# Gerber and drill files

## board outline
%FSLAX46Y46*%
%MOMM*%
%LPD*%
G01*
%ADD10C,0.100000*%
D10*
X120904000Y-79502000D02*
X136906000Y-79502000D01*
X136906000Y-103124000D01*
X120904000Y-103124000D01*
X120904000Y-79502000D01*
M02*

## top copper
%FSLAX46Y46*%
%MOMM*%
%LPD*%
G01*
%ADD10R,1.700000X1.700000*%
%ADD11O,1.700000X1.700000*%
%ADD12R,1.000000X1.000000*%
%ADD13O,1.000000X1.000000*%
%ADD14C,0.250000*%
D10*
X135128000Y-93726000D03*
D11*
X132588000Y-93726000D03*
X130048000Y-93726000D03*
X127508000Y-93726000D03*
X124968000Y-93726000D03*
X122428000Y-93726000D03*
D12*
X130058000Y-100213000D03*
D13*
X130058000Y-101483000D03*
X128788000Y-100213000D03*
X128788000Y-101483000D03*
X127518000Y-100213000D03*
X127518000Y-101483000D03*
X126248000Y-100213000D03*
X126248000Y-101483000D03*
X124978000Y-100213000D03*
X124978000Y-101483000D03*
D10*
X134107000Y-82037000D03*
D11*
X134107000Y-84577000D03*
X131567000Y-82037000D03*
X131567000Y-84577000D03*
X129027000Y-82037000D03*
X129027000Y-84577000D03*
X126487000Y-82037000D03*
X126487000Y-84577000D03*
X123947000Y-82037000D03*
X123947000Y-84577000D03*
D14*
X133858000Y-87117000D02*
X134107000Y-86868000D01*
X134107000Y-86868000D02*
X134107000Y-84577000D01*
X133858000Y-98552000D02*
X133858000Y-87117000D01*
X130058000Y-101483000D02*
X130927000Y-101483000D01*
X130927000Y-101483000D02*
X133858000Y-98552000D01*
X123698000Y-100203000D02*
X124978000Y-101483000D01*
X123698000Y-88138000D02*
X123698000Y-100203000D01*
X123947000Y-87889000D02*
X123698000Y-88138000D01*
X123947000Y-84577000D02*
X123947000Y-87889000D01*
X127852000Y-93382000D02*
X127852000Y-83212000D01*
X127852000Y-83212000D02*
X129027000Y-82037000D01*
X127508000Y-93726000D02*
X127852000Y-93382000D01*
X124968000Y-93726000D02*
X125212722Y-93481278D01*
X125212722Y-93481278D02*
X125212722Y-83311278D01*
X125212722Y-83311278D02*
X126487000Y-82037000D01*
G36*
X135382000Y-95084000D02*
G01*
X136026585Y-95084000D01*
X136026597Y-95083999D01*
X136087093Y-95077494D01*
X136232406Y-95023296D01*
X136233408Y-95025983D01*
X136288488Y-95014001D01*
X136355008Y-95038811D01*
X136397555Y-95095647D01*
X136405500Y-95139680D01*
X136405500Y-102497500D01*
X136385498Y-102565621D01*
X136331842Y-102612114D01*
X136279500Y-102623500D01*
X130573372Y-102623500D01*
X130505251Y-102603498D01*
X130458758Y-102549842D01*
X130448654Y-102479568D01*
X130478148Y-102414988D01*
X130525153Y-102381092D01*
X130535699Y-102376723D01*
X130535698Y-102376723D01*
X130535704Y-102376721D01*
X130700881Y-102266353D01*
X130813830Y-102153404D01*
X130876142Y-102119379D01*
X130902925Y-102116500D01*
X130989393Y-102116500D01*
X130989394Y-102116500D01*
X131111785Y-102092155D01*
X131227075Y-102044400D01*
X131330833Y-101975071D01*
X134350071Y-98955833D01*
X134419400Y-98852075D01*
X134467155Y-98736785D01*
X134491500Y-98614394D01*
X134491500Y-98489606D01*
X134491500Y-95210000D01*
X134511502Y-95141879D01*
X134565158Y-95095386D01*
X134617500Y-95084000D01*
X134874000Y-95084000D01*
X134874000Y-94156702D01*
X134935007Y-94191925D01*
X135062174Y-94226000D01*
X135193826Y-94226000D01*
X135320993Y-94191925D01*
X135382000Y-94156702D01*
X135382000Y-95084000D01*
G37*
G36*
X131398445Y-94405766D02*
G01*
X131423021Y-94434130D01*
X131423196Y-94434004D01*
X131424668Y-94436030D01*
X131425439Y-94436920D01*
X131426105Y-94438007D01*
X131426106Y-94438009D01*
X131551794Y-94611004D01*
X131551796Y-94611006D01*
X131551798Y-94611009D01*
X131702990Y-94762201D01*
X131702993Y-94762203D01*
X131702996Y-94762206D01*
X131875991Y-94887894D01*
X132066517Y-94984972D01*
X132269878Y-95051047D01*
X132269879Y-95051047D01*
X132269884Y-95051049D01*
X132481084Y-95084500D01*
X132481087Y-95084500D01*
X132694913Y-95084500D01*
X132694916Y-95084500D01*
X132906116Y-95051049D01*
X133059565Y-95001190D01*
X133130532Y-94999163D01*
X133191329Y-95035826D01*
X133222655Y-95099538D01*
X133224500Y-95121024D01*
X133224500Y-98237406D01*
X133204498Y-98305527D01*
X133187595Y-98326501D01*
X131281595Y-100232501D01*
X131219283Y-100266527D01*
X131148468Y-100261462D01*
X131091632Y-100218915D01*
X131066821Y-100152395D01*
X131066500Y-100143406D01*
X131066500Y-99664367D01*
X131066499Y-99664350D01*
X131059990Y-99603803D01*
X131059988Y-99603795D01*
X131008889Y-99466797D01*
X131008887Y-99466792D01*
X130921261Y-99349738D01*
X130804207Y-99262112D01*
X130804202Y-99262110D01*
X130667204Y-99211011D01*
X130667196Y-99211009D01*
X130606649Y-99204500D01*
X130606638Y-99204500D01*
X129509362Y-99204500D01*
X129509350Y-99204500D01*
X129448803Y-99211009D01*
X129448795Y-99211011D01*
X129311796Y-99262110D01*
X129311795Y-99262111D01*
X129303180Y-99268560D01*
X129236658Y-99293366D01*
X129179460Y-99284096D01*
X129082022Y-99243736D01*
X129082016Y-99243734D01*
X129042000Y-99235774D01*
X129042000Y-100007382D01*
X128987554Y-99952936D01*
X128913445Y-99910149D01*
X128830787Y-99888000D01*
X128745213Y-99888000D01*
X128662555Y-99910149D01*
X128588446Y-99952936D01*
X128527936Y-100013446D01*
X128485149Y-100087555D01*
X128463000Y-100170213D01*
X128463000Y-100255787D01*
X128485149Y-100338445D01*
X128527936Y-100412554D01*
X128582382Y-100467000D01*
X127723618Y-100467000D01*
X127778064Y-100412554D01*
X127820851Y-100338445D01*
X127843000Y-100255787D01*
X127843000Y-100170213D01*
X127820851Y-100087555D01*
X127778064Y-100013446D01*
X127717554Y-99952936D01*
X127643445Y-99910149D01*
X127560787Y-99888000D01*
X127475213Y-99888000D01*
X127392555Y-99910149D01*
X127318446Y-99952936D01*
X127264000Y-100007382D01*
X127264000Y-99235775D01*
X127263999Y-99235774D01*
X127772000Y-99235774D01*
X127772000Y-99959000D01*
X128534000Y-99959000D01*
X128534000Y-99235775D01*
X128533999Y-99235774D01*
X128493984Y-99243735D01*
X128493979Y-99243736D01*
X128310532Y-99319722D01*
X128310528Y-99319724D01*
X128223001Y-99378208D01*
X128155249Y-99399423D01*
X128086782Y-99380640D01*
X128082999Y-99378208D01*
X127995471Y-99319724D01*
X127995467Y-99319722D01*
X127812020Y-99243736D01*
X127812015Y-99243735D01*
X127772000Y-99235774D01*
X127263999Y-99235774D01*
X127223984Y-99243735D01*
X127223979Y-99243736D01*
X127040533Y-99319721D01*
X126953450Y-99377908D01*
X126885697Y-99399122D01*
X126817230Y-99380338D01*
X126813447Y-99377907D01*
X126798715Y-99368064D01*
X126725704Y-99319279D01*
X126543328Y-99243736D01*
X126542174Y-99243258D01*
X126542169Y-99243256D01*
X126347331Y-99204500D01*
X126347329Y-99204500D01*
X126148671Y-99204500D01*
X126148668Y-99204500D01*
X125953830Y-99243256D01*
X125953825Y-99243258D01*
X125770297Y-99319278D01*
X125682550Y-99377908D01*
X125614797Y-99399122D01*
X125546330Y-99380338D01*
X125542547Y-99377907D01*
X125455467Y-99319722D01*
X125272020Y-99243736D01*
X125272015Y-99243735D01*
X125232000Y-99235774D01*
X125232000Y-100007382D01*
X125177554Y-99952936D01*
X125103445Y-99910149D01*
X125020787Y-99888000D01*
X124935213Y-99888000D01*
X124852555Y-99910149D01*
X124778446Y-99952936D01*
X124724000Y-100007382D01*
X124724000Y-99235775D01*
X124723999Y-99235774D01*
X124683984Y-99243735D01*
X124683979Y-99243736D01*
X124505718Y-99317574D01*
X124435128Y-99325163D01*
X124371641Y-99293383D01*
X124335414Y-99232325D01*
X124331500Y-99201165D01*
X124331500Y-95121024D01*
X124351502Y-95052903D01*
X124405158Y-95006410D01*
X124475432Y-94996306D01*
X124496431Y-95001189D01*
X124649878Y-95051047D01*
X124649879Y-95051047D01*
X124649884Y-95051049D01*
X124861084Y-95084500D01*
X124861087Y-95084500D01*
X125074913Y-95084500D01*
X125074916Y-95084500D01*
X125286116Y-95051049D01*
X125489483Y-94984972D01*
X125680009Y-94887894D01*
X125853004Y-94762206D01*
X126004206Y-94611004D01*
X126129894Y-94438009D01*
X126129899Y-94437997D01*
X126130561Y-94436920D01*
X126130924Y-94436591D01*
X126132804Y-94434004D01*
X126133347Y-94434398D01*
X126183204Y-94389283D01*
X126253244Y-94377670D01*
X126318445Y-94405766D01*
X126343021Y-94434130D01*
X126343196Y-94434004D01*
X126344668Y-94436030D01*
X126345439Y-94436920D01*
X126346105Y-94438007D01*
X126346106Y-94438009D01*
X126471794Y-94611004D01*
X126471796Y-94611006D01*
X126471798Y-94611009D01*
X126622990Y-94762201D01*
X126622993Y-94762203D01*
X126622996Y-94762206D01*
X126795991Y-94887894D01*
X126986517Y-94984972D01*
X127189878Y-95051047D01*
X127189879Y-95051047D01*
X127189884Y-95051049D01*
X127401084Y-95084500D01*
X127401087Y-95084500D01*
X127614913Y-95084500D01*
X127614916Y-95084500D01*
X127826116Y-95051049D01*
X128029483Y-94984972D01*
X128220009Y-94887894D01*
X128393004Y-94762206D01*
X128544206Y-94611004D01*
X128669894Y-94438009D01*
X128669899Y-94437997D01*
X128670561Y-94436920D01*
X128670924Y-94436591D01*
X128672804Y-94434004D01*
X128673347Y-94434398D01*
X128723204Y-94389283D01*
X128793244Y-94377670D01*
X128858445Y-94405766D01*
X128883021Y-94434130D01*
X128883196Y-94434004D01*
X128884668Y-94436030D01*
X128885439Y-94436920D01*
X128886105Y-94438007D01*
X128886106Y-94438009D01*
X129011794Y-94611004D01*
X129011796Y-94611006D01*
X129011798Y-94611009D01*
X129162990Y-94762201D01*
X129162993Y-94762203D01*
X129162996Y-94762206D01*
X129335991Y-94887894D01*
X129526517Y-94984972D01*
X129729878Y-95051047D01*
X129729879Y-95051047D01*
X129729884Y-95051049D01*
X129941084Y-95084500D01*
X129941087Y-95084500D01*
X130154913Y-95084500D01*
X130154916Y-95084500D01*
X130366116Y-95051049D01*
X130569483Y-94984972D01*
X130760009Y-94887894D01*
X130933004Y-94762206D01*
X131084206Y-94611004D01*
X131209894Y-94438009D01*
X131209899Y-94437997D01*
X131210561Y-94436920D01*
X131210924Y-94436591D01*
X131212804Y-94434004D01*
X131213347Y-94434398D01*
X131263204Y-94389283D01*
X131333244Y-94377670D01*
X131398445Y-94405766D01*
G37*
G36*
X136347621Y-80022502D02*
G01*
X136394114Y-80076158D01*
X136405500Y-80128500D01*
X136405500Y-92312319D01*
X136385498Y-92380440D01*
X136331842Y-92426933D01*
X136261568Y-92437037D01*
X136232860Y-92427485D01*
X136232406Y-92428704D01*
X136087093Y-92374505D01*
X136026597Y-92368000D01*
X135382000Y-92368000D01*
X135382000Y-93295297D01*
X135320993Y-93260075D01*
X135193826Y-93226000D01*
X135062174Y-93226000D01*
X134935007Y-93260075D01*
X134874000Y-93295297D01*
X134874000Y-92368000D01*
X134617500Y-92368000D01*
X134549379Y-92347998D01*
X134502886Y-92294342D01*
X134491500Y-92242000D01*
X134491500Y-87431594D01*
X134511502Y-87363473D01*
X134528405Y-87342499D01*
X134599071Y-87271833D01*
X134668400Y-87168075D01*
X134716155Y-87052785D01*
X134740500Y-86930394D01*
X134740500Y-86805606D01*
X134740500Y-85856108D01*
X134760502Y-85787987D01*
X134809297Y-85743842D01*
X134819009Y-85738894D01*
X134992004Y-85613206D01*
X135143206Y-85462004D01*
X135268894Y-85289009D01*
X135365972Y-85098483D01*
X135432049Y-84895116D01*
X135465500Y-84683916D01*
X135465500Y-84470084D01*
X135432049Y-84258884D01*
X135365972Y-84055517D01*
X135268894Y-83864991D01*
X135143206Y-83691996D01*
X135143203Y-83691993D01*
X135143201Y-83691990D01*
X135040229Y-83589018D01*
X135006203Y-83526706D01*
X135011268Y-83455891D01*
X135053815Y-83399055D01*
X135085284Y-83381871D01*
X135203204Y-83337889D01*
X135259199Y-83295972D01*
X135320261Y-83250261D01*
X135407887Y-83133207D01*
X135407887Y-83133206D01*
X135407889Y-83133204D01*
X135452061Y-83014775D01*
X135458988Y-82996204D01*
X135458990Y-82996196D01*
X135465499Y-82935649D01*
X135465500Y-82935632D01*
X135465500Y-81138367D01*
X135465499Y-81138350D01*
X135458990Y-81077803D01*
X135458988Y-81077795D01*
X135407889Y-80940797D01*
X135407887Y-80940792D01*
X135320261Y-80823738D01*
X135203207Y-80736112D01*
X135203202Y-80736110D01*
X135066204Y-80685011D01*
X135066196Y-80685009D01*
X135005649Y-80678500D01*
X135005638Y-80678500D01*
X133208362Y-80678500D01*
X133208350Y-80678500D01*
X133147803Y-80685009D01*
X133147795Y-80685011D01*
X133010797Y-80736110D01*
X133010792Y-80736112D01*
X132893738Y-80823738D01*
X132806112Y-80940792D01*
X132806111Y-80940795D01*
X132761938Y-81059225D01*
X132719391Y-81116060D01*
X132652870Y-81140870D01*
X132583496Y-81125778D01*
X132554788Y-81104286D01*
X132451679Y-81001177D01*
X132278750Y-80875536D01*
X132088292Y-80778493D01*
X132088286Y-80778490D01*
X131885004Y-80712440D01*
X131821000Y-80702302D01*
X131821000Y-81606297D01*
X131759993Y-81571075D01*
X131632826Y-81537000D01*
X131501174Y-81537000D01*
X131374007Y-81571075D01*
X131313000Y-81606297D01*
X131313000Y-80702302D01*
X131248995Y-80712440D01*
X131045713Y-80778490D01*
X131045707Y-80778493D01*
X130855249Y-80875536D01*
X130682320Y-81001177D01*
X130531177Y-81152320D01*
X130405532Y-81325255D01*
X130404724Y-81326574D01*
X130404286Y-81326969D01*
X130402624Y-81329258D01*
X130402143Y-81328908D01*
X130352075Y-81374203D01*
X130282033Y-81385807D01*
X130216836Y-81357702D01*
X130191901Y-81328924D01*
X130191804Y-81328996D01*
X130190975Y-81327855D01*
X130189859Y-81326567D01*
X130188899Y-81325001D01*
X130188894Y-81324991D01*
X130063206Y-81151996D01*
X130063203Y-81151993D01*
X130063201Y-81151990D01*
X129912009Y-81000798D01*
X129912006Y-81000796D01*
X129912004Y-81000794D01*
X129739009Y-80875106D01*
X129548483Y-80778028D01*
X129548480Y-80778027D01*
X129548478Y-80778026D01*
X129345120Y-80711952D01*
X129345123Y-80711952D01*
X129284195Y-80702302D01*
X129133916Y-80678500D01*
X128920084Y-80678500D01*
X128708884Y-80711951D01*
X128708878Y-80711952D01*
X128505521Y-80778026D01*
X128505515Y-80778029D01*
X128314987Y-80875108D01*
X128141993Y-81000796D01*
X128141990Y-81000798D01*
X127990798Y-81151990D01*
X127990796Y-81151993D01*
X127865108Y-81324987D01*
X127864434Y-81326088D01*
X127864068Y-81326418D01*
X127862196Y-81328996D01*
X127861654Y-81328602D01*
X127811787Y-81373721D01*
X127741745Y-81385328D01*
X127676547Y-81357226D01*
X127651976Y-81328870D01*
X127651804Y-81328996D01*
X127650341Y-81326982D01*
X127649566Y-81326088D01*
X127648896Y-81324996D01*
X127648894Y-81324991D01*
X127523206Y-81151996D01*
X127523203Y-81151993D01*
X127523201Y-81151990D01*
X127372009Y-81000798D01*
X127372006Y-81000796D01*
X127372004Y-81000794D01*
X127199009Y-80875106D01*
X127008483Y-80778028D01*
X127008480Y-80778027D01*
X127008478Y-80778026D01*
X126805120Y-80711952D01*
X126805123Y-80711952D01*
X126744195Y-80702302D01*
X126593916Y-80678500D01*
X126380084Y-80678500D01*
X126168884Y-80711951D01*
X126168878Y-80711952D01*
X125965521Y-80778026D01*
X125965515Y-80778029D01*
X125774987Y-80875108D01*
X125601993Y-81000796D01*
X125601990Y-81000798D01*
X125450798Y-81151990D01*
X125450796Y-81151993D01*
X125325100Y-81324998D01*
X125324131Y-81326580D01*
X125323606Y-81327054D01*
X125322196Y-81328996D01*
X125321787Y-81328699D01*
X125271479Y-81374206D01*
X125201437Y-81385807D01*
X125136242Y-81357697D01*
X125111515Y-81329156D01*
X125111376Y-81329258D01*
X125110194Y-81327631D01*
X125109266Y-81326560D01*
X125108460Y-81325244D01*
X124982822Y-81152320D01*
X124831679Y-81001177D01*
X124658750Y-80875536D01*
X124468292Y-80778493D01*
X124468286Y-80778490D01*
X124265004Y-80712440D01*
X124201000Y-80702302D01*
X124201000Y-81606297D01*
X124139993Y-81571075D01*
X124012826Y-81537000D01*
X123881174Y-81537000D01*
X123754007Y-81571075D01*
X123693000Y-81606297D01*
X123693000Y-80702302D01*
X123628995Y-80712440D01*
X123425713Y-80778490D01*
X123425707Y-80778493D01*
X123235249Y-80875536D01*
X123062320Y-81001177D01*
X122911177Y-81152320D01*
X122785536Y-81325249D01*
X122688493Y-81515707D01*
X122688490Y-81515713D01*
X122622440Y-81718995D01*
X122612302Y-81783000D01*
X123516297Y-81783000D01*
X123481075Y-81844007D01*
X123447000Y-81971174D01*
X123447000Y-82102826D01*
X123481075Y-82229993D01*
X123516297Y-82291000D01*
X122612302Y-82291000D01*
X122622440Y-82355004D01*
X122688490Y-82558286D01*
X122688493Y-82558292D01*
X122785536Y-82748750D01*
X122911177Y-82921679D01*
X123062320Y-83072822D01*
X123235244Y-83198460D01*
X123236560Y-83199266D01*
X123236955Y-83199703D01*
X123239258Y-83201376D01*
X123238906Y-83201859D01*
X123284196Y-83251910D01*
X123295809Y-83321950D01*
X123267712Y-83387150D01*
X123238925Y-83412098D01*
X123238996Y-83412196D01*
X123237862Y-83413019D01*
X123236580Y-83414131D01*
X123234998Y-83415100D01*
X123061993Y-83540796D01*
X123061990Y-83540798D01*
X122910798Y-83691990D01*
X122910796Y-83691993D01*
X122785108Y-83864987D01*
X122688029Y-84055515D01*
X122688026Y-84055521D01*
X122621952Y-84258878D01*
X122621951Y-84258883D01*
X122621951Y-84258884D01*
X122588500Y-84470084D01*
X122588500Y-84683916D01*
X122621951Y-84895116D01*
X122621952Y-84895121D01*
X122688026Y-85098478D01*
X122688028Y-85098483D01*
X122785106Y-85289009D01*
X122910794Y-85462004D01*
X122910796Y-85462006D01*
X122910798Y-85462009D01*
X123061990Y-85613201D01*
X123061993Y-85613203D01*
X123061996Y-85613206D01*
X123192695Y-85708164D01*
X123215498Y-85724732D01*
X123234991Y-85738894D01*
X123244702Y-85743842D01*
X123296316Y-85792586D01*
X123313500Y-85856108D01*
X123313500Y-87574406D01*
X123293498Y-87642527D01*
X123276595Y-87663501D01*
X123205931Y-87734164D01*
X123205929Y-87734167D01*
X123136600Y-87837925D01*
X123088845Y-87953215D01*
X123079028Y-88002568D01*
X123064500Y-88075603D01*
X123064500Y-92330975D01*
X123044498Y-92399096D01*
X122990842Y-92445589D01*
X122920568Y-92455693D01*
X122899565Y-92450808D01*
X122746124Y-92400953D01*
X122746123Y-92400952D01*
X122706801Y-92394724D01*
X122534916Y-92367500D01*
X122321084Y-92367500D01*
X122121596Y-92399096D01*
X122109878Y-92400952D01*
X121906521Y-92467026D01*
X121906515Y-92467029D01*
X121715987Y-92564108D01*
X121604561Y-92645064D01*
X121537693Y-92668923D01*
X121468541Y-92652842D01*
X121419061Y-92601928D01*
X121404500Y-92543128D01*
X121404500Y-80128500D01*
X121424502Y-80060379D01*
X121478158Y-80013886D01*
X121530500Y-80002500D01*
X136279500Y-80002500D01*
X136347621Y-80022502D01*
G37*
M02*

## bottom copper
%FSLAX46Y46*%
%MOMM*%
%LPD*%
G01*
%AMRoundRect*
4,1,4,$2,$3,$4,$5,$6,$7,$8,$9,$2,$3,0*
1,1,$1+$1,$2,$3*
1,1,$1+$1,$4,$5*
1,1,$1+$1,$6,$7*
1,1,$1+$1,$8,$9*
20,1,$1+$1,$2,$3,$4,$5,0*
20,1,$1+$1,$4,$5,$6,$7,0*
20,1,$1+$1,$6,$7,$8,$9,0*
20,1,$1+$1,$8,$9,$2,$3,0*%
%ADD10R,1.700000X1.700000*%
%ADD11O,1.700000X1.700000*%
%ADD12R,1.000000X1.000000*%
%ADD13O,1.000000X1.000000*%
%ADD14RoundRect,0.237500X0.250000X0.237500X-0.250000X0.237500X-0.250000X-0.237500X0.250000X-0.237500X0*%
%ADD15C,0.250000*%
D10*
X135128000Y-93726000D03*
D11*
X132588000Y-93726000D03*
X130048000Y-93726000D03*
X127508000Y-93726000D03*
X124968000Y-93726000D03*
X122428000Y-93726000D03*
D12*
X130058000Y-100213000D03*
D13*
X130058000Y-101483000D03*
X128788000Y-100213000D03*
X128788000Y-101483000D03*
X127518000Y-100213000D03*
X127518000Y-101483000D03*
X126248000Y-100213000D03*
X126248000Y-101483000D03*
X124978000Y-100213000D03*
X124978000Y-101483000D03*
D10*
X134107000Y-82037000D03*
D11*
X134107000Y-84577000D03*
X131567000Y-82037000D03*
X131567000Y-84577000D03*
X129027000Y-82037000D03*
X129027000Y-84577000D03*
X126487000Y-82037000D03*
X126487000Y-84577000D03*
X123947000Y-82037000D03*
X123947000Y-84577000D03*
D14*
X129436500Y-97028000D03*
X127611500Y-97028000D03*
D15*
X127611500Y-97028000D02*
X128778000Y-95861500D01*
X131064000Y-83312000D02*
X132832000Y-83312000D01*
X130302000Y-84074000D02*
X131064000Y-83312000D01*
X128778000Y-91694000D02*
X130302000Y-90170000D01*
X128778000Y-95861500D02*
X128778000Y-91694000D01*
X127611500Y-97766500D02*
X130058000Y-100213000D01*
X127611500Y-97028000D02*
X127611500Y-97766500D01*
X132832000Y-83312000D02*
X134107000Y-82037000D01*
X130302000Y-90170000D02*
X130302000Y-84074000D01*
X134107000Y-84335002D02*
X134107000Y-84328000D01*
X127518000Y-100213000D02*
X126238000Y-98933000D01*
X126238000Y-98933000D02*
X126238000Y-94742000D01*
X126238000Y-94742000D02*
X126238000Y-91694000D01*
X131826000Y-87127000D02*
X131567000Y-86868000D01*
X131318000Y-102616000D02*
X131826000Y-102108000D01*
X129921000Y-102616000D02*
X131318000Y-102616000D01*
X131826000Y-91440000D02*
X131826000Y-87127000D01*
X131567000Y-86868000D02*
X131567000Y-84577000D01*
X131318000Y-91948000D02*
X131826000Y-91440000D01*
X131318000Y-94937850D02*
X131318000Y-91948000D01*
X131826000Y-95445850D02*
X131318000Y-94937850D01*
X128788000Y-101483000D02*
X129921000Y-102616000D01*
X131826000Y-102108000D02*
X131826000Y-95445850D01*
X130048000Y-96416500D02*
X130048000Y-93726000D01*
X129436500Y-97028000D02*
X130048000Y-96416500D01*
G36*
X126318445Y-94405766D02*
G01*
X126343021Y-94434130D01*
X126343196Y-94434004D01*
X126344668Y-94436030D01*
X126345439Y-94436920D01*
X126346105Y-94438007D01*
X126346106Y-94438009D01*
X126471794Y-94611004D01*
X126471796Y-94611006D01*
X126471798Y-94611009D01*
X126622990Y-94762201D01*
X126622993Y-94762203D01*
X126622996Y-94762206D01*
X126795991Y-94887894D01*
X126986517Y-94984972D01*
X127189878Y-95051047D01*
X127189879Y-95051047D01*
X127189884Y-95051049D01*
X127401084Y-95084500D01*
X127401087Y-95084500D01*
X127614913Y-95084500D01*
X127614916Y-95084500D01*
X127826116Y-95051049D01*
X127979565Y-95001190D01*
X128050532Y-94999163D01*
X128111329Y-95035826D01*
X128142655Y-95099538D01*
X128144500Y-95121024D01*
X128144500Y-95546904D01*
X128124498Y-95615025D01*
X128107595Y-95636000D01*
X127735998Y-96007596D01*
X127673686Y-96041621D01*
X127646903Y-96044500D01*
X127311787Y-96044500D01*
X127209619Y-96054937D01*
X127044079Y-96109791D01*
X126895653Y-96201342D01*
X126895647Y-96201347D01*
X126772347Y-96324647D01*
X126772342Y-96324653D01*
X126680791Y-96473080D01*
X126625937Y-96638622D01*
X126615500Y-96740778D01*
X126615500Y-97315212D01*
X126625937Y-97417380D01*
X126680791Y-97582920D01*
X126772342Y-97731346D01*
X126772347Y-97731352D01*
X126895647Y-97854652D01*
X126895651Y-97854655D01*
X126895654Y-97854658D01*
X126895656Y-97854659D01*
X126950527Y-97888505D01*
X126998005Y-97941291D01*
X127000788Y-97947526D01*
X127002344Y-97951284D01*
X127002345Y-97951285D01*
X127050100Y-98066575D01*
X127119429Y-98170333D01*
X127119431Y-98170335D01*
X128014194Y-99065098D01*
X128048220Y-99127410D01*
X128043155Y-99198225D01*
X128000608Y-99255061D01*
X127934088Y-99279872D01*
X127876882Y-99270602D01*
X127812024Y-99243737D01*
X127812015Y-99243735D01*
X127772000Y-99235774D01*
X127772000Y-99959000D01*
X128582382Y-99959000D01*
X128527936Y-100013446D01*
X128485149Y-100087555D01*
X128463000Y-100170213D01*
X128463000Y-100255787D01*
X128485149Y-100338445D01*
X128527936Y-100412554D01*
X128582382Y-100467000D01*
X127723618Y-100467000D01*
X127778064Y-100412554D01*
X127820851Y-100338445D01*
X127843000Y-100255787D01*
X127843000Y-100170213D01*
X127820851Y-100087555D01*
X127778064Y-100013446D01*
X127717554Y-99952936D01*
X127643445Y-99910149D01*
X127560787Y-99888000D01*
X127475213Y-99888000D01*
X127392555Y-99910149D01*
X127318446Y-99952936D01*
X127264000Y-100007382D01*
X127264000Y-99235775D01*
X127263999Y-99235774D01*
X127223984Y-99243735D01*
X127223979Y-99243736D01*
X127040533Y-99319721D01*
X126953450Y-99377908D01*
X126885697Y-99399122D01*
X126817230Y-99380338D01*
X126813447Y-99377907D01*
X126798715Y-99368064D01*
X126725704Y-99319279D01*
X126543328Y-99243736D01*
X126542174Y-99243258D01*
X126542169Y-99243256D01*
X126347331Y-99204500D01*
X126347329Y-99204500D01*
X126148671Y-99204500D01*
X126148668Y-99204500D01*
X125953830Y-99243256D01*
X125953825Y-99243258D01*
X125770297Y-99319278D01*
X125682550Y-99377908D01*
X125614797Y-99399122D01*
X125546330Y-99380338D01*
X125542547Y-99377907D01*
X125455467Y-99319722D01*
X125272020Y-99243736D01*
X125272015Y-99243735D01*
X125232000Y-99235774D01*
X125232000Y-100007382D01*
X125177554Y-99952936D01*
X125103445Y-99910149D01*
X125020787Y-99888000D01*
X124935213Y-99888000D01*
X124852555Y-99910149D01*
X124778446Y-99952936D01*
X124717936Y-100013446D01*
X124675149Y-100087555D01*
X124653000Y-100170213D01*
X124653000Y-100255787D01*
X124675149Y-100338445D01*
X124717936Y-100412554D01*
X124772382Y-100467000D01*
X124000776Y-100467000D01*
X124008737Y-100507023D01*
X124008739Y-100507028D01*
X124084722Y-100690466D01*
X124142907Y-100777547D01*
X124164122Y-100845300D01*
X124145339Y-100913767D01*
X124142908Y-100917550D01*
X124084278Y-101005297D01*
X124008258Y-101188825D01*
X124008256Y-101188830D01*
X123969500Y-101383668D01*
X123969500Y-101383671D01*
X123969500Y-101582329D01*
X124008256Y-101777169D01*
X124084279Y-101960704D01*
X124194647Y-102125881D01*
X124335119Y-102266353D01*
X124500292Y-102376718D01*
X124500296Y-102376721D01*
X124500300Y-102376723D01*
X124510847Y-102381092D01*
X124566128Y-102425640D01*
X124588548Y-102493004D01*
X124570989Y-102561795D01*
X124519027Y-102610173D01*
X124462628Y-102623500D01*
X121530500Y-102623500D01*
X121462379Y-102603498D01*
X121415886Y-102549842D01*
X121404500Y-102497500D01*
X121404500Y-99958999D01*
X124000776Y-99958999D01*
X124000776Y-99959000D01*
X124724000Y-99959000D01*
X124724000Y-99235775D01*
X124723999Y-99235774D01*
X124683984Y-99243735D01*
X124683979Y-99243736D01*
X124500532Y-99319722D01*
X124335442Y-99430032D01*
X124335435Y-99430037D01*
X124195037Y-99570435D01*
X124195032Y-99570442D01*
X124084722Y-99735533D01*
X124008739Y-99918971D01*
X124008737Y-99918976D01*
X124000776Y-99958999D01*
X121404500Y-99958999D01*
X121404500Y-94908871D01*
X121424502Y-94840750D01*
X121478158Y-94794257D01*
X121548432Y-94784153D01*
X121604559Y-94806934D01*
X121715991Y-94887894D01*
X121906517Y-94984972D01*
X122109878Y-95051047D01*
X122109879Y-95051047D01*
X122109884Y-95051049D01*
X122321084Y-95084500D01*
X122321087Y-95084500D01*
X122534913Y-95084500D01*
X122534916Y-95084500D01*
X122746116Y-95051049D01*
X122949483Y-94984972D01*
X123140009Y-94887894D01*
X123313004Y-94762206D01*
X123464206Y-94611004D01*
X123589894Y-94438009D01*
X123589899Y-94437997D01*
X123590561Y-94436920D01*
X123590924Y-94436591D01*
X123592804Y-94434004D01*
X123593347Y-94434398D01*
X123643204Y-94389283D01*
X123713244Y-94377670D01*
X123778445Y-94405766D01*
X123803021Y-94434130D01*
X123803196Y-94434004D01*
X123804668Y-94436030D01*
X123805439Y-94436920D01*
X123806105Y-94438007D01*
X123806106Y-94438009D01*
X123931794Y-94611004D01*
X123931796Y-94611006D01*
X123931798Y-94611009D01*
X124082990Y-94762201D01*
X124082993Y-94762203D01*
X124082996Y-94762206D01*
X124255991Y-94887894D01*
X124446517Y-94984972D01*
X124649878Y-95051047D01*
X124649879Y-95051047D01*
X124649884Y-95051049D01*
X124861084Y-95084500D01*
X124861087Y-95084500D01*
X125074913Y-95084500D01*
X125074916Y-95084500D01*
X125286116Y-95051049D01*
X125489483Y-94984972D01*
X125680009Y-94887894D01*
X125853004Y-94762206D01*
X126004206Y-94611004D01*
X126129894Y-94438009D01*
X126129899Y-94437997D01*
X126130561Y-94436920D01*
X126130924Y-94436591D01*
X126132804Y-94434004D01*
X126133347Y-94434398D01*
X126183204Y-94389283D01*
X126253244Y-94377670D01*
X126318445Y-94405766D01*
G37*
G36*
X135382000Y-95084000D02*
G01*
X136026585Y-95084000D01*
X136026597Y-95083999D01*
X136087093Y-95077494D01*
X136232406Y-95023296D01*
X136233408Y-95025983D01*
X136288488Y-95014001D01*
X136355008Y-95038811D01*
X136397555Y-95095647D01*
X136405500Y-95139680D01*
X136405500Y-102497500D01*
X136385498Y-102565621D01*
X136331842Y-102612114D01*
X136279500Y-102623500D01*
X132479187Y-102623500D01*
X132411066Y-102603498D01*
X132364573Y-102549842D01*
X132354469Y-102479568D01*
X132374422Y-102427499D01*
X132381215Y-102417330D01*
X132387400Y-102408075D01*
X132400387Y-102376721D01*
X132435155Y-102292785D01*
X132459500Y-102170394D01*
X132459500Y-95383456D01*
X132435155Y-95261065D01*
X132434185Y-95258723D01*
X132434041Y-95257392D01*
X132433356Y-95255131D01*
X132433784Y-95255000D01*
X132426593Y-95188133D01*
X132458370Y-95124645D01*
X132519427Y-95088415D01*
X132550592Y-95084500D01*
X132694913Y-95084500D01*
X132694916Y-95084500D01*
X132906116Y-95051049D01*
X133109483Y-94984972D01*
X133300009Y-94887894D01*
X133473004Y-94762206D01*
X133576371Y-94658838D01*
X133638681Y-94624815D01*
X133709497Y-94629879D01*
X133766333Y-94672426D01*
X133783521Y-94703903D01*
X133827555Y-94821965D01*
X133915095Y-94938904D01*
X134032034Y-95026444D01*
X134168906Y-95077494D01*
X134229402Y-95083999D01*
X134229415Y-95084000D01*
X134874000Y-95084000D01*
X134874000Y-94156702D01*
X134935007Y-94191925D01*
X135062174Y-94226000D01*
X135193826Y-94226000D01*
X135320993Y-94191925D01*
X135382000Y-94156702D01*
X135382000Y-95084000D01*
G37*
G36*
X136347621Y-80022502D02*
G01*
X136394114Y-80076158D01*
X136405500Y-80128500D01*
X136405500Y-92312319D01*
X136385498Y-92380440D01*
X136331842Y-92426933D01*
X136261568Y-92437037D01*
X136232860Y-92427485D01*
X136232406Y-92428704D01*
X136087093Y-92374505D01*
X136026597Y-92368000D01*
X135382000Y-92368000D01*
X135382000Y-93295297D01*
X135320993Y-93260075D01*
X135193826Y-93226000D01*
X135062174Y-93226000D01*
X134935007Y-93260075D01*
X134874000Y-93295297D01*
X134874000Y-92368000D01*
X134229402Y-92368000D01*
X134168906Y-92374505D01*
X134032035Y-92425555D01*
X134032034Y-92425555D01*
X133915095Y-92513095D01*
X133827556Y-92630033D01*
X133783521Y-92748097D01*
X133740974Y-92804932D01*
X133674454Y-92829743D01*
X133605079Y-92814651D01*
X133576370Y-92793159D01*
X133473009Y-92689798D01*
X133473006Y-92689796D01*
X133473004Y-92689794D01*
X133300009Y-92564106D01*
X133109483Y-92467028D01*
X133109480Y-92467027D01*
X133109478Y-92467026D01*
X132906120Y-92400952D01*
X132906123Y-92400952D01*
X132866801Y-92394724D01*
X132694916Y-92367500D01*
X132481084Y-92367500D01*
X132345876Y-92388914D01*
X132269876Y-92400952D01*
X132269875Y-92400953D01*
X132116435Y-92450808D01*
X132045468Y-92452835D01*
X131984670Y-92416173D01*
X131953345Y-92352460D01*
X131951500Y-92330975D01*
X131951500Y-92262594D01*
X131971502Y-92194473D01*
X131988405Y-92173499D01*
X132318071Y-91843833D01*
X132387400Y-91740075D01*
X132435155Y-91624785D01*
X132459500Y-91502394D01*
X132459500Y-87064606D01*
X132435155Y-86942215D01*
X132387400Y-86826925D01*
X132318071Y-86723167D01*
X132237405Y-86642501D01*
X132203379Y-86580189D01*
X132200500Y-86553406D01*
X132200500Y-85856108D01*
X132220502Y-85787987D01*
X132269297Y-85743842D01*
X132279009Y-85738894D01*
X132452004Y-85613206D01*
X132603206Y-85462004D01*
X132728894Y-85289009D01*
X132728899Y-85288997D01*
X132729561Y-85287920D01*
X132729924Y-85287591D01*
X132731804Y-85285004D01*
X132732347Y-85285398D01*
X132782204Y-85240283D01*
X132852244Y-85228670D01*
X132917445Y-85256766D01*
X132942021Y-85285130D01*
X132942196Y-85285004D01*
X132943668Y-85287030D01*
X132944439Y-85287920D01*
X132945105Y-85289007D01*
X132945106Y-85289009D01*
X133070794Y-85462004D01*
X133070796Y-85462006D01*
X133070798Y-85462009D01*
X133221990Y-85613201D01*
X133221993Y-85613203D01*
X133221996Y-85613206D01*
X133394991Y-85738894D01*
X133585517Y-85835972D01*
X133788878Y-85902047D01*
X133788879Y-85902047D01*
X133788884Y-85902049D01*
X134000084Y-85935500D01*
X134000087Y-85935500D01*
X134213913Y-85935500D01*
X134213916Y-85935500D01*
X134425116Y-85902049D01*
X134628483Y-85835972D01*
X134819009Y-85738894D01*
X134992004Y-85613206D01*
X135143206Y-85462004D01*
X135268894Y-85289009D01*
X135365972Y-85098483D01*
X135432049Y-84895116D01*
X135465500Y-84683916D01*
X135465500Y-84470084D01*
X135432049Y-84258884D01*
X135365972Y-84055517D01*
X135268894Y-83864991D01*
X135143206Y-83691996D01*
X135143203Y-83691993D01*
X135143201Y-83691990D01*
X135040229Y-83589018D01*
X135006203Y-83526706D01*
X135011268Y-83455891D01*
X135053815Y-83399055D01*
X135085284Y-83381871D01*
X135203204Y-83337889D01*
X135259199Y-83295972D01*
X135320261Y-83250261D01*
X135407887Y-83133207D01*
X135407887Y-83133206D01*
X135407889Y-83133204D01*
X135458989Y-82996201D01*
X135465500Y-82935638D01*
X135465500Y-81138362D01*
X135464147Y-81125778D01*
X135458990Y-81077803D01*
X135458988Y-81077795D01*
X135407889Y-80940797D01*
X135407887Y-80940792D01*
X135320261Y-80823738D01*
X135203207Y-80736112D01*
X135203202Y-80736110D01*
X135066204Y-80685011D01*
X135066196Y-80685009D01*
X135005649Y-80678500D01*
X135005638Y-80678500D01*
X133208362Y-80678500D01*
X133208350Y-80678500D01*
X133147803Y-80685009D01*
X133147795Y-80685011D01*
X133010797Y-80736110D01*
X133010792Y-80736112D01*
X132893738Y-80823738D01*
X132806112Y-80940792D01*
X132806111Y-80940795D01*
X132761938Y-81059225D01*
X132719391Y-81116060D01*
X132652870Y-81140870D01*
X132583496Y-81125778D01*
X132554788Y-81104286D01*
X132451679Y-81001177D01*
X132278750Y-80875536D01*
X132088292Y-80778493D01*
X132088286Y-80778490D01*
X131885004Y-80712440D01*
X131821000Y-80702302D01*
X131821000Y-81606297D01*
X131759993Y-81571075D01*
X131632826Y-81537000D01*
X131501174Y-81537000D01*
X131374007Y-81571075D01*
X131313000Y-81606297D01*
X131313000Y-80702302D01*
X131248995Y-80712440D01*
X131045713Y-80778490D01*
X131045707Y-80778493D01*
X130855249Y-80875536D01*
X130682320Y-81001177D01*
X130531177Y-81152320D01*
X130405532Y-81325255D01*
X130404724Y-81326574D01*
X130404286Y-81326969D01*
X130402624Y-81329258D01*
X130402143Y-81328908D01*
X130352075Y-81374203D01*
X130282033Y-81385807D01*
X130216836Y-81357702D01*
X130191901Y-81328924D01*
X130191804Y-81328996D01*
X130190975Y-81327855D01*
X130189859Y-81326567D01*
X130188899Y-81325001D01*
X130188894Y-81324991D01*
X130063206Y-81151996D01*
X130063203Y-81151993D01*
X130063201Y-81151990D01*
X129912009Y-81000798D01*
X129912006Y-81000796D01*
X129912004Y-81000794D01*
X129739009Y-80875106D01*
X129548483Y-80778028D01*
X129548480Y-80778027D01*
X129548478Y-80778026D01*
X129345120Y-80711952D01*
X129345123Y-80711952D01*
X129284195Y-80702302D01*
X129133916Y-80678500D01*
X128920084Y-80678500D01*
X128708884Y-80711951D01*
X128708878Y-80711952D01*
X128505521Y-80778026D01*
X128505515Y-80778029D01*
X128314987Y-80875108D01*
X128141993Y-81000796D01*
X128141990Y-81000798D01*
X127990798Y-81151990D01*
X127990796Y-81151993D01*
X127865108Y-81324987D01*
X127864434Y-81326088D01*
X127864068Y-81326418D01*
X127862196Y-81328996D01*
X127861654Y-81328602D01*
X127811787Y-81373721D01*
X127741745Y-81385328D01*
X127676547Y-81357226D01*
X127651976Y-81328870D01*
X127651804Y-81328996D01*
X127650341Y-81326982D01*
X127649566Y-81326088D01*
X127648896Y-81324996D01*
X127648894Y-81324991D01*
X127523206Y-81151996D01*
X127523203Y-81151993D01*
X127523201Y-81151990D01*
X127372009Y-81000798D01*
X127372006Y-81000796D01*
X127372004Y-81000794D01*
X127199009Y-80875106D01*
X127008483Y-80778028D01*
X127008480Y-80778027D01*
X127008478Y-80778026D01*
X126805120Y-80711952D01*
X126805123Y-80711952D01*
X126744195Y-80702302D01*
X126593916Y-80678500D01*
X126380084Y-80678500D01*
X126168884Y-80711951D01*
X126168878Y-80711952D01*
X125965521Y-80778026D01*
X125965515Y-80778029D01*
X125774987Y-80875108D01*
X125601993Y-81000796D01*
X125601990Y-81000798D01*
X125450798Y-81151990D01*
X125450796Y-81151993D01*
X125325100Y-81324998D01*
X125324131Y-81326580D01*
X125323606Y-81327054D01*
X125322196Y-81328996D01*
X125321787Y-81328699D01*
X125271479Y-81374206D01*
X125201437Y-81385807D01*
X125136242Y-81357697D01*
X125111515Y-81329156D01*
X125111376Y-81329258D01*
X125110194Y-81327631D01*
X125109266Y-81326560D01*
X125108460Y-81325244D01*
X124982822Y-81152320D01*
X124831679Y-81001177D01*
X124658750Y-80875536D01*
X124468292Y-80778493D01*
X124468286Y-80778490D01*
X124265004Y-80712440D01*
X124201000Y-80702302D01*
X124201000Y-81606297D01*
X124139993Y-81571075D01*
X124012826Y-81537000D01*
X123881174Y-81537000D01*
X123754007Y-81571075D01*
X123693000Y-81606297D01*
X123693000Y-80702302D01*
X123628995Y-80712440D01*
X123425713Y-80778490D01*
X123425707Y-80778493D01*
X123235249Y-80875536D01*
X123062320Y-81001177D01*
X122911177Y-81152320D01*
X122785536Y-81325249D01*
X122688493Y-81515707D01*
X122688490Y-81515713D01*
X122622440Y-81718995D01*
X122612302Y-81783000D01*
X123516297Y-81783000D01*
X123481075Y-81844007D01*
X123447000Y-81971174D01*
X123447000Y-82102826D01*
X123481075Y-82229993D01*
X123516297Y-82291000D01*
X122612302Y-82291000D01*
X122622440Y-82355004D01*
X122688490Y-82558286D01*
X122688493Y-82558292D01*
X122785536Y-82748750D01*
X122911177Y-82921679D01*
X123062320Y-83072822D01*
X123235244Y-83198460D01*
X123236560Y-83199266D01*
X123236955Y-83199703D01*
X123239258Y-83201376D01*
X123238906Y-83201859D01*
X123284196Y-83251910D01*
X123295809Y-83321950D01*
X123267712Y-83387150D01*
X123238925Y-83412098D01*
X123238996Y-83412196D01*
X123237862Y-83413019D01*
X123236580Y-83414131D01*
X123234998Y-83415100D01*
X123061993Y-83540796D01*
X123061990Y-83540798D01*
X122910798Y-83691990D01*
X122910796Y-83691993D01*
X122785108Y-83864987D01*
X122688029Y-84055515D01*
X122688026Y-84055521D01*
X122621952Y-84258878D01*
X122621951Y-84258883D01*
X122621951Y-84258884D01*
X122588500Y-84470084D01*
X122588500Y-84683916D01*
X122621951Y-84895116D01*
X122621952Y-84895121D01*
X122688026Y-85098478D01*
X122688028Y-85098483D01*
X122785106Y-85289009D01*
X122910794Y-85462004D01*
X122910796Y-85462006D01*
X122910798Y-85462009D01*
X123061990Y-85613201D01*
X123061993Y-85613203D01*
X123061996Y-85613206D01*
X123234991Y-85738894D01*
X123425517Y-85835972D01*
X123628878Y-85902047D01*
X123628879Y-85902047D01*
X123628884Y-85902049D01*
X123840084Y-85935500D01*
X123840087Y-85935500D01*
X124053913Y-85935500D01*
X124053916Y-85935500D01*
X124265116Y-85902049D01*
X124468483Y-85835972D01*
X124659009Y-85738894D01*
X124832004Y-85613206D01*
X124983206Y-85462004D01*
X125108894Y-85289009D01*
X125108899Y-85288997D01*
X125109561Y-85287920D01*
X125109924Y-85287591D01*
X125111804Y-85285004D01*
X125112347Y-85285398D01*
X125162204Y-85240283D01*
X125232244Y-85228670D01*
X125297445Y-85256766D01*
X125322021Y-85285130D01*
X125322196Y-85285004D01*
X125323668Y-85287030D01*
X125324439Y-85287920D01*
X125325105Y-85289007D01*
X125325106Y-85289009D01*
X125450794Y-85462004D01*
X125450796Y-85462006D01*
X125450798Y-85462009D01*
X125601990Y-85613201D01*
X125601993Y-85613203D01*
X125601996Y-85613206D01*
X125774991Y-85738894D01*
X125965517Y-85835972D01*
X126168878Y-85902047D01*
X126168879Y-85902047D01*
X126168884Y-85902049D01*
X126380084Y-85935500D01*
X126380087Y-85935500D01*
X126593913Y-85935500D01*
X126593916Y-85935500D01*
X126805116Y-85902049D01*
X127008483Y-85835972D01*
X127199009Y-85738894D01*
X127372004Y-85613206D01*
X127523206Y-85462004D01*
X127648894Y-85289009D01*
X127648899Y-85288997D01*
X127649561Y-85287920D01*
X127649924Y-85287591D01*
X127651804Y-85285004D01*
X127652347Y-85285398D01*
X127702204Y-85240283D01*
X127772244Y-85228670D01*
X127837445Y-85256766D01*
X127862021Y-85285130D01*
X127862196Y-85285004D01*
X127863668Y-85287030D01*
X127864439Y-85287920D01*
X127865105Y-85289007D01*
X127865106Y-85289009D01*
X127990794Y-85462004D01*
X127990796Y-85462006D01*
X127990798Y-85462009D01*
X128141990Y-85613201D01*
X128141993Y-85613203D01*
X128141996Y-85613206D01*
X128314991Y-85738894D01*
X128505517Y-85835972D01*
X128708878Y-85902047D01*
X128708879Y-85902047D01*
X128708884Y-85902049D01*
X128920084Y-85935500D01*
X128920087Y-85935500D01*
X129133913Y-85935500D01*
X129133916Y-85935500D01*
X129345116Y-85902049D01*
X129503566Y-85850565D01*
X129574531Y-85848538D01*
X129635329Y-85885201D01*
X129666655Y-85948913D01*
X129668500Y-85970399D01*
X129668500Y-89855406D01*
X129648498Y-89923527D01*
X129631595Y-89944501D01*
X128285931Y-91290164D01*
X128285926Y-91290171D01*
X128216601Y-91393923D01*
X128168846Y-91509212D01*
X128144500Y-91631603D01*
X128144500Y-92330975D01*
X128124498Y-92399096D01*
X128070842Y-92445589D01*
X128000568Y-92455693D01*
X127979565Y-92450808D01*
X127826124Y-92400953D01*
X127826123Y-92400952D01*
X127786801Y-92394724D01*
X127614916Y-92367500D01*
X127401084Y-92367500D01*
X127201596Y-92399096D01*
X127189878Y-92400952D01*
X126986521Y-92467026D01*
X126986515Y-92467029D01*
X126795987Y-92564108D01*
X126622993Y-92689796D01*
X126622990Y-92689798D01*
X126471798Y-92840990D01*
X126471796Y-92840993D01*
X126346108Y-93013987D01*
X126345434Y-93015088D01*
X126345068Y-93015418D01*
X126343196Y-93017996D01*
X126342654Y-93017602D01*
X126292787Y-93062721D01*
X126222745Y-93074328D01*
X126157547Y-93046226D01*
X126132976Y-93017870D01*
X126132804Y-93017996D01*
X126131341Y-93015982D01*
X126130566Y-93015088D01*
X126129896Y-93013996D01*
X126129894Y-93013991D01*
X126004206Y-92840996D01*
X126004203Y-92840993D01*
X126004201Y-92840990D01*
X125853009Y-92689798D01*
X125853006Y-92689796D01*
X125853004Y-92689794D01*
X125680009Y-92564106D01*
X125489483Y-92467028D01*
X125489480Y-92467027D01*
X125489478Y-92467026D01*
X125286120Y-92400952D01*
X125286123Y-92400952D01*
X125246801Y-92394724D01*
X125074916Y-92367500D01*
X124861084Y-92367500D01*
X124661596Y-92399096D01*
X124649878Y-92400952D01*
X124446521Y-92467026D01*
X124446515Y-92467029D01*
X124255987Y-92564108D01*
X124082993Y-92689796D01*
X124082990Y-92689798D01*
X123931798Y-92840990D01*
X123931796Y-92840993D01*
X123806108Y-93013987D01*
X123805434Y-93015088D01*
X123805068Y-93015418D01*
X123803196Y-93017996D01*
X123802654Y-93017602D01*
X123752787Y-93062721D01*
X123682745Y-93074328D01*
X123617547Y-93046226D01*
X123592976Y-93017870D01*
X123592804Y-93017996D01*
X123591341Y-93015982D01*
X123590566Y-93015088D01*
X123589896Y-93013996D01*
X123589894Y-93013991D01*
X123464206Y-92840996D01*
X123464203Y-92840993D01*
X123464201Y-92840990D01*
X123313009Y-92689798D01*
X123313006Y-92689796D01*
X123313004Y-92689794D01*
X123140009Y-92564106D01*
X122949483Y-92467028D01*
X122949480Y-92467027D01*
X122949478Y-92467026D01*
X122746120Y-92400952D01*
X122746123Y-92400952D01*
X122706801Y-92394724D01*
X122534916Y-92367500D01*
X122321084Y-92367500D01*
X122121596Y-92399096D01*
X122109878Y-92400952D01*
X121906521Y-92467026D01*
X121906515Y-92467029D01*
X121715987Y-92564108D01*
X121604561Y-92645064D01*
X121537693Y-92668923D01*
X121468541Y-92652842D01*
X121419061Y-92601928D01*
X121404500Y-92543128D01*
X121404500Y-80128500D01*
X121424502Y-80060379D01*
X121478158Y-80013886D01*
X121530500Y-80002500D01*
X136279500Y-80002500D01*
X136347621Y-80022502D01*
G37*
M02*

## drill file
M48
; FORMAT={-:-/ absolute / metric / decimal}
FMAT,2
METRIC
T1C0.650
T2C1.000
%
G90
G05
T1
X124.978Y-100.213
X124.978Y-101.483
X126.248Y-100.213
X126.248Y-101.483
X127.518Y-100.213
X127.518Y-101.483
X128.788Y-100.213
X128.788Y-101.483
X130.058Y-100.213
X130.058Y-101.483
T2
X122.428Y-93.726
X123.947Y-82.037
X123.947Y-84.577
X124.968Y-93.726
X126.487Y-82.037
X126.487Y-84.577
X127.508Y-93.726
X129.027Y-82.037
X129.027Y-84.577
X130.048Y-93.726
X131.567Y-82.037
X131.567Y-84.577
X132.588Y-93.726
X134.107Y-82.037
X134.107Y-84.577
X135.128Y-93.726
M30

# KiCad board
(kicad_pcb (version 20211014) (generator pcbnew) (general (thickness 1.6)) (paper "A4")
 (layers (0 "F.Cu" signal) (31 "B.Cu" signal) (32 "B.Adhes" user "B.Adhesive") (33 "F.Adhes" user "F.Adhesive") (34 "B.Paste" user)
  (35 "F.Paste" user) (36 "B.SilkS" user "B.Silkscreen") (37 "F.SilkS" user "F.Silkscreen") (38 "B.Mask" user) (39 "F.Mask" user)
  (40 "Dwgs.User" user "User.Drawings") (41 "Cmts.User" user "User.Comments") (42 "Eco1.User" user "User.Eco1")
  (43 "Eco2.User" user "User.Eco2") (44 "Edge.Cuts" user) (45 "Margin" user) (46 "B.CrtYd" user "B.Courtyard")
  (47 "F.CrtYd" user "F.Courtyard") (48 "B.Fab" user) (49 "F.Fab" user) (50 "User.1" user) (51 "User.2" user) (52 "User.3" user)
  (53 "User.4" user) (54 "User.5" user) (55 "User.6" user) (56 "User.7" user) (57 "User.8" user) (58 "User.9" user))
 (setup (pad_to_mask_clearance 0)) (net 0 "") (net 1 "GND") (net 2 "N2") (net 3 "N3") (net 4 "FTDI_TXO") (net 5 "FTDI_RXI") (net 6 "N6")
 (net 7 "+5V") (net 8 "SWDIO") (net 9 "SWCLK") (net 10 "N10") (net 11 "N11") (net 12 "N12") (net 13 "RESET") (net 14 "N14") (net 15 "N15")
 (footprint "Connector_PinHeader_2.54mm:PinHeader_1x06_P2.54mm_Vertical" (layer "F.Cu") (at 135.128 93.726 -90)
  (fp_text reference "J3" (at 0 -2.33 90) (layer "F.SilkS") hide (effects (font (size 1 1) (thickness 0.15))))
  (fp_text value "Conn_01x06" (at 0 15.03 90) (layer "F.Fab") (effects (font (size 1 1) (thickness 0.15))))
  (pad "1" thru_hole rect (at 0 0 270) (size 1.7 1.7) (drill 1) (layers *.Cu *.Mask) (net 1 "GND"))
  (pad "2" thru_hole oval (at 0 2.54 270) (size 1.7 1.7) (drill 1) (layers *.Cu *.Mask) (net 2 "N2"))
  (pad "3" thru_hole oval (at 0 5.08 270) (size 1.7 1.7) (drill 1) (layers *.Cu *.Mask) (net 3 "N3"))
  (pad "4" thru_hole oval (at 0 7.62 270) (size 1.7 1.7) (drill 1) (layers *.Cu *.Mask) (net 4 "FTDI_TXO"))
  (pad "5" thru_hole oval (at 0 10.16 270) (size 1.7 1.7) (drill 1) (layers *.Cu *.Mask) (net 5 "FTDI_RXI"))
  (pad "6" thru_hole oval (at 0 12.7 270) (size 1.7 1.7) (drill 1) (layers *.Cu *.Mask) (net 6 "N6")))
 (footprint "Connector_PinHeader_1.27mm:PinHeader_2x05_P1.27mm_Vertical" (layer "F.Cu") (at 130.058 100.213 -90)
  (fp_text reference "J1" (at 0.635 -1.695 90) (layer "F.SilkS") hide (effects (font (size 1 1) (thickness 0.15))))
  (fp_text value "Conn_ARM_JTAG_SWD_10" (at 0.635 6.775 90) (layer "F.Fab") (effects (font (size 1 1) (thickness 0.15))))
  (pad "1" thru_hole rect (at 0 0 270) (size 1 1) (drill 0.65) (layers *.Cu *.Mask) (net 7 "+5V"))
  (pad "2" thru_hole oval (at 1.27 0 270) (size 1 1) (drill 0.65) (layers *.Cu *.Mask) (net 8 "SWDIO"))
  (pad "3" thru_hole oval (at 0 1.27 270) (size 1 1) (drill 0.65) (layers *.Cu *.Mask) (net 1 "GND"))
  (pad "4" thru_hole oval (at 1.27 1.27 270) (size 1 1) (drill 0.65) (layers *.Cu *.Mask) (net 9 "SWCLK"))
  (pad "5" thru_hole oval (at 0 2.54 270) (size 1 1) (drill 0.65) (layers *.Cu *.Mask) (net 1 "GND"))
  (pad "6" thru_hole oval (at 1.27 2.54 270) (size 1 1) (drill 0.65) (layers *.Cu *.Mask) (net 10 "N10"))
  (pad "7" thru_hole oval (at 0 3.81 270) (size 1 1) (drill 0.65) (layers *.Cu *.Mask) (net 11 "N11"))
  (pad "8" thru_hole oval (at 1.27 3.81 270) (size 1 1) (drill 0.65) (layers *.Cu *.Mask) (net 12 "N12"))
  (pad "9" thru_hole oval (at 0 5.08 270) (size 1 1) (drill 0.65) (layers *.Cu *.Mask) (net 1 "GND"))
  (pad "10" thru_hole oval (at 1.27 5.08 270) (size 1 1) (drill 0.65) (layers *.Cu *.Mask) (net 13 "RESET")))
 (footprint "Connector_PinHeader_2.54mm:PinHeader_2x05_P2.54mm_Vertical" (layer "F.Cu") (at 134.107 82.037 -90)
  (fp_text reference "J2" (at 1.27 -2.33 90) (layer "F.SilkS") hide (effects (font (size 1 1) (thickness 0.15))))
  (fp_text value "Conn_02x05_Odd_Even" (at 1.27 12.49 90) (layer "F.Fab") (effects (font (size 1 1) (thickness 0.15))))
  (pad "1" thru_hole rect (at 0 0 270) (size 1.7 1.7) (drill 1) (layers *.Cu *.Mask) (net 7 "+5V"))
  (pad "2" thru_hole oval (at 2.54 0 270) (size 1.7 1.7) (drill 1) (layers *.Cu *.Mask) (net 8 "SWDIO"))
  (pad "3" thru_hole oval (at 0 2.54 270) (size 1.7 1.7) (drill 1) (layers *.Cu *.Mask) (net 1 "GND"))
  (pad "4" thru_hole oval (at 2.54 2.54 270) (size 1.7 1.7) (drill 1) (layers *.Cu *.Mask) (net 9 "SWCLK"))
  (pad "5" thru_hole oval (at 0 5.08 270) (size 1.7 1.7) (drill 1) (layers *.Cu *.Mask) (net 4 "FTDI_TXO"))
  (pad "6" thru_hole oval (at 2.54 5.08 270) (size 1.7 1.7) (drill 1) (layers *.Cu *.Mask) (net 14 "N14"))
  (pad "7" thru_hole oval (at 0 7.62 270) (size 1.7 1.7) (drill 1) (layers *.Cu *.Mask) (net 5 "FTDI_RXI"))
  (pad "8" thru_hole oval (at 2.54 7.62 270) (size 1.7 1.7) (drill 1) (layers *.Cu *.Mask) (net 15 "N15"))
  (pad "9" thru_hole oval (at 0 10.16 270) (size 1.7 1.7) (drill 1) (layers *.Cu *.Mask) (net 1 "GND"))
  (pad "10" thru_hole oval (at 2.54 10.16 270) (size 1.7 1.7) (drill 1) (layers *.Cu *.Mask) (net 13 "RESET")))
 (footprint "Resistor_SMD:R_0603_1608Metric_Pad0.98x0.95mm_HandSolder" (layer "B.Cu") (at 128.524 97.028 180)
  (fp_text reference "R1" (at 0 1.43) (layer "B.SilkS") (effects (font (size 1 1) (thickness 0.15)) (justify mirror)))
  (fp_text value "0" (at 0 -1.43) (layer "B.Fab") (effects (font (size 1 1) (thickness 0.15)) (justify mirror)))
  (pad "1" smd roundrect (at -0.9125 0 180) (size 0.975 0.95) (layers "B.Cu" "B.Paste" "B.Mask") (roundrect_rratio 0.25) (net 3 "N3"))
  (pad "2" smd roundrect (at 0.9125 0 180) (size 0.975 0.95) (layers "B.Cu" "B.Paste" "B.Mask") (roundrect_rratio 0.25) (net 7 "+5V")))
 (gr_rect (start 136.906 103.124) (end 120.904 79.502) (layer "Edge.Cuts") (width 0.1) (fill none))
 (segment (start 127.6115 97.028) (end 128.778 95.8615) (width 0.25) (layer "B.Cu") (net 7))
 (segment (start 131.064 83.312) (end 132.832 83.312) (width 0.25) (layer "B.Cu") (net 7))
 (segment (start 130.302 84.074) (end 131.064 83.312) (width 0.25) (layer "B.Cu") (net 7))
 (segment (start 128.778 91.694) (end 130.302 90.17) (width 0.25) (layer "B.Cu") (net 7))
 (segment (start 128.778 95.8615) (end 128.778 91.694) (width 0.25) (layer "B.Cu") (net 7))
 (segment (start 127.6115 97.7665) (end 130.058 100.213) (width 0.25) (layer "B.Cu") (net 7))
 (segment (start 127.6115 97.028) (end 127.6115 97.7665) (width 0.25) (layer "B.Cu") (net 7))
 (segment (start 132.832 83.312) (end 134.107 82.037) (width 0.25) (layer "B.Cu") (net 7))
 (segment (start 130.302 90.17) (end 130.302 84.074) (width 0.25) (layer "B.Cu") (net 7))
 (segment (start 133.858 87.117) (end 134.107 86.868) (width 0.25) (layer "F.Cu") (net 8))
 (segment (start 134.107 86.868) (end 134.107 84.577) (width 0.25) (layer "F.Cu") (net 8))
 (segment (start 133.858 98.552) (end 133.858 87.117) (width 0.25) (layer "F.Cu") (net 8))
 (segment (start 130.058 101.483) (end 130.927 101.483) (width 0.25) (layer "F.Cu") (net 8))
 (segment (start 130.927 101.483) (end 133.858 98.552) (width 0.25) (layer "F.Cu") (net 8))
 (segment (start 134.107 84.335002) (end 134.107 84.328) (width 0.25) (layer "B.Cu") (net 8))
 (segment (start 127.518 100.213) (end 126.238 98.933) (width 0.25) (layer "B.Cu") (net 1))
 (segment (start 126.238 98.933) (end 126.238 94.742) (width 0.25) (layer "B.Cu") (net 1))
 (segment (start 126.238 94.742) (end 126.238 91.694) (width 0.25) (layer "B.Cu") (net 1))
 (segment (start 131.826 87.127) (end 131.567 86.868) (width 0.25) (layer "B.Cu") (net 9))
 (segment (start 131.318 102.616) (end 131.826 102.108) (width 0.25) (layer "B.Cu") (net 9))
 (segment (start 129.921 102.616) (end 131.318 102.616) (width 0.25) (layer "B.Cu") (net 9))
 (segment (start 131.826 91.44) (end 131.826 87.127) (width 0.25) (layer "B.Cu") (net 9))
 (segment (start 131.567 86.868) (end 131.567 84.577) (width 0.25) (layer "B.Cu") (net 9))
 (segment (start 131.318 91.948) (end 131.826 91.44) (width 0.25) (layer "B.Cu") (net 9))
 (segment (start 131.318 94.93785) (end 131.318 91.948) (width 0.25) (layer "B.Cu") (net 9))
 (segment (start 131.826 95.44585) (end 131.318 94.93785) (width 0.25) (layer "B.Cu") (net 9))
 (segment (start 128.788 101.483) (end 129.921 102.616) (width 0.25) (layer "B.Cu") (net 9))
 (segment (start 131.826 102.108) (end 131.826 95.44585) (width 0.25) (layer "B.Cu") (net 9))
 (segment (start 123.698 100.203) (end 124.978 101.483) (width 0.25) (layer "F.Cu") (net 13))
 (segment (start 123.698 88.138) (end 123.698 100.203) (width 0.25) (layer "F.Cu") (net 13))
 (segment (start 123.947 87.889) (end 123.698 88.138) (width 0.25) (layer "F.Cu") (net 13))
 (segment (start 123.947 84.577) (end 123.947 87.889) (width 0.25) (layer "F.Cu") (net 13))
 (segment (start 127.852 93.382) (end 127.852 83.212) (width 0.25) (layer "F.Cu") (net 4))
 (segment (start 127.852 83.212) (end 129.027 82.037) (width 0.25) (layer "F.Cu") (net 4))
 (segment (start 127.508 93.726) (end 127.852 93.382) (width 0.25) (layer "F.Cu") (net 4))
 (segment (start 124.968 93.726) (end 125.212722 93.481278) (width 0.25) (layer "F.Cu") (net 5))
 (segment (start 125.212722 93.481278) (end 125.212722 83.311278) (width 0.25) (layer "F.Cu") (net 5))
 (segment (start 125.212722 83.311278) (end 126.487 82.037) (width 0.25) (layer "F.Cu") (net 5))
 (segment (start 130.048 96.4165) (end 130.048 93.726) (width 0.25) (layer "B.Cu") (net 3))
 (segment (start 129.4365 97.028) (end 130.048 96.4165) (width 0.25) (layer "B.Cu") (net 3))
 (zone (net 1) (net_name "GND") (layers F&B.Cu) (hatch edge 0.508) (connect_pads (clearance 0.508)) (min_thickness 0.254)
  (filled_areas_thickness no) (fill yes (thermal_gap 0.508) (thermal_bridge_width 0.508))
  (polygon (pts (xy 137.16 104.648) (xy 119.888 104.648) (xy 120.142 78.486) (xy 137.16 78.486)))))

